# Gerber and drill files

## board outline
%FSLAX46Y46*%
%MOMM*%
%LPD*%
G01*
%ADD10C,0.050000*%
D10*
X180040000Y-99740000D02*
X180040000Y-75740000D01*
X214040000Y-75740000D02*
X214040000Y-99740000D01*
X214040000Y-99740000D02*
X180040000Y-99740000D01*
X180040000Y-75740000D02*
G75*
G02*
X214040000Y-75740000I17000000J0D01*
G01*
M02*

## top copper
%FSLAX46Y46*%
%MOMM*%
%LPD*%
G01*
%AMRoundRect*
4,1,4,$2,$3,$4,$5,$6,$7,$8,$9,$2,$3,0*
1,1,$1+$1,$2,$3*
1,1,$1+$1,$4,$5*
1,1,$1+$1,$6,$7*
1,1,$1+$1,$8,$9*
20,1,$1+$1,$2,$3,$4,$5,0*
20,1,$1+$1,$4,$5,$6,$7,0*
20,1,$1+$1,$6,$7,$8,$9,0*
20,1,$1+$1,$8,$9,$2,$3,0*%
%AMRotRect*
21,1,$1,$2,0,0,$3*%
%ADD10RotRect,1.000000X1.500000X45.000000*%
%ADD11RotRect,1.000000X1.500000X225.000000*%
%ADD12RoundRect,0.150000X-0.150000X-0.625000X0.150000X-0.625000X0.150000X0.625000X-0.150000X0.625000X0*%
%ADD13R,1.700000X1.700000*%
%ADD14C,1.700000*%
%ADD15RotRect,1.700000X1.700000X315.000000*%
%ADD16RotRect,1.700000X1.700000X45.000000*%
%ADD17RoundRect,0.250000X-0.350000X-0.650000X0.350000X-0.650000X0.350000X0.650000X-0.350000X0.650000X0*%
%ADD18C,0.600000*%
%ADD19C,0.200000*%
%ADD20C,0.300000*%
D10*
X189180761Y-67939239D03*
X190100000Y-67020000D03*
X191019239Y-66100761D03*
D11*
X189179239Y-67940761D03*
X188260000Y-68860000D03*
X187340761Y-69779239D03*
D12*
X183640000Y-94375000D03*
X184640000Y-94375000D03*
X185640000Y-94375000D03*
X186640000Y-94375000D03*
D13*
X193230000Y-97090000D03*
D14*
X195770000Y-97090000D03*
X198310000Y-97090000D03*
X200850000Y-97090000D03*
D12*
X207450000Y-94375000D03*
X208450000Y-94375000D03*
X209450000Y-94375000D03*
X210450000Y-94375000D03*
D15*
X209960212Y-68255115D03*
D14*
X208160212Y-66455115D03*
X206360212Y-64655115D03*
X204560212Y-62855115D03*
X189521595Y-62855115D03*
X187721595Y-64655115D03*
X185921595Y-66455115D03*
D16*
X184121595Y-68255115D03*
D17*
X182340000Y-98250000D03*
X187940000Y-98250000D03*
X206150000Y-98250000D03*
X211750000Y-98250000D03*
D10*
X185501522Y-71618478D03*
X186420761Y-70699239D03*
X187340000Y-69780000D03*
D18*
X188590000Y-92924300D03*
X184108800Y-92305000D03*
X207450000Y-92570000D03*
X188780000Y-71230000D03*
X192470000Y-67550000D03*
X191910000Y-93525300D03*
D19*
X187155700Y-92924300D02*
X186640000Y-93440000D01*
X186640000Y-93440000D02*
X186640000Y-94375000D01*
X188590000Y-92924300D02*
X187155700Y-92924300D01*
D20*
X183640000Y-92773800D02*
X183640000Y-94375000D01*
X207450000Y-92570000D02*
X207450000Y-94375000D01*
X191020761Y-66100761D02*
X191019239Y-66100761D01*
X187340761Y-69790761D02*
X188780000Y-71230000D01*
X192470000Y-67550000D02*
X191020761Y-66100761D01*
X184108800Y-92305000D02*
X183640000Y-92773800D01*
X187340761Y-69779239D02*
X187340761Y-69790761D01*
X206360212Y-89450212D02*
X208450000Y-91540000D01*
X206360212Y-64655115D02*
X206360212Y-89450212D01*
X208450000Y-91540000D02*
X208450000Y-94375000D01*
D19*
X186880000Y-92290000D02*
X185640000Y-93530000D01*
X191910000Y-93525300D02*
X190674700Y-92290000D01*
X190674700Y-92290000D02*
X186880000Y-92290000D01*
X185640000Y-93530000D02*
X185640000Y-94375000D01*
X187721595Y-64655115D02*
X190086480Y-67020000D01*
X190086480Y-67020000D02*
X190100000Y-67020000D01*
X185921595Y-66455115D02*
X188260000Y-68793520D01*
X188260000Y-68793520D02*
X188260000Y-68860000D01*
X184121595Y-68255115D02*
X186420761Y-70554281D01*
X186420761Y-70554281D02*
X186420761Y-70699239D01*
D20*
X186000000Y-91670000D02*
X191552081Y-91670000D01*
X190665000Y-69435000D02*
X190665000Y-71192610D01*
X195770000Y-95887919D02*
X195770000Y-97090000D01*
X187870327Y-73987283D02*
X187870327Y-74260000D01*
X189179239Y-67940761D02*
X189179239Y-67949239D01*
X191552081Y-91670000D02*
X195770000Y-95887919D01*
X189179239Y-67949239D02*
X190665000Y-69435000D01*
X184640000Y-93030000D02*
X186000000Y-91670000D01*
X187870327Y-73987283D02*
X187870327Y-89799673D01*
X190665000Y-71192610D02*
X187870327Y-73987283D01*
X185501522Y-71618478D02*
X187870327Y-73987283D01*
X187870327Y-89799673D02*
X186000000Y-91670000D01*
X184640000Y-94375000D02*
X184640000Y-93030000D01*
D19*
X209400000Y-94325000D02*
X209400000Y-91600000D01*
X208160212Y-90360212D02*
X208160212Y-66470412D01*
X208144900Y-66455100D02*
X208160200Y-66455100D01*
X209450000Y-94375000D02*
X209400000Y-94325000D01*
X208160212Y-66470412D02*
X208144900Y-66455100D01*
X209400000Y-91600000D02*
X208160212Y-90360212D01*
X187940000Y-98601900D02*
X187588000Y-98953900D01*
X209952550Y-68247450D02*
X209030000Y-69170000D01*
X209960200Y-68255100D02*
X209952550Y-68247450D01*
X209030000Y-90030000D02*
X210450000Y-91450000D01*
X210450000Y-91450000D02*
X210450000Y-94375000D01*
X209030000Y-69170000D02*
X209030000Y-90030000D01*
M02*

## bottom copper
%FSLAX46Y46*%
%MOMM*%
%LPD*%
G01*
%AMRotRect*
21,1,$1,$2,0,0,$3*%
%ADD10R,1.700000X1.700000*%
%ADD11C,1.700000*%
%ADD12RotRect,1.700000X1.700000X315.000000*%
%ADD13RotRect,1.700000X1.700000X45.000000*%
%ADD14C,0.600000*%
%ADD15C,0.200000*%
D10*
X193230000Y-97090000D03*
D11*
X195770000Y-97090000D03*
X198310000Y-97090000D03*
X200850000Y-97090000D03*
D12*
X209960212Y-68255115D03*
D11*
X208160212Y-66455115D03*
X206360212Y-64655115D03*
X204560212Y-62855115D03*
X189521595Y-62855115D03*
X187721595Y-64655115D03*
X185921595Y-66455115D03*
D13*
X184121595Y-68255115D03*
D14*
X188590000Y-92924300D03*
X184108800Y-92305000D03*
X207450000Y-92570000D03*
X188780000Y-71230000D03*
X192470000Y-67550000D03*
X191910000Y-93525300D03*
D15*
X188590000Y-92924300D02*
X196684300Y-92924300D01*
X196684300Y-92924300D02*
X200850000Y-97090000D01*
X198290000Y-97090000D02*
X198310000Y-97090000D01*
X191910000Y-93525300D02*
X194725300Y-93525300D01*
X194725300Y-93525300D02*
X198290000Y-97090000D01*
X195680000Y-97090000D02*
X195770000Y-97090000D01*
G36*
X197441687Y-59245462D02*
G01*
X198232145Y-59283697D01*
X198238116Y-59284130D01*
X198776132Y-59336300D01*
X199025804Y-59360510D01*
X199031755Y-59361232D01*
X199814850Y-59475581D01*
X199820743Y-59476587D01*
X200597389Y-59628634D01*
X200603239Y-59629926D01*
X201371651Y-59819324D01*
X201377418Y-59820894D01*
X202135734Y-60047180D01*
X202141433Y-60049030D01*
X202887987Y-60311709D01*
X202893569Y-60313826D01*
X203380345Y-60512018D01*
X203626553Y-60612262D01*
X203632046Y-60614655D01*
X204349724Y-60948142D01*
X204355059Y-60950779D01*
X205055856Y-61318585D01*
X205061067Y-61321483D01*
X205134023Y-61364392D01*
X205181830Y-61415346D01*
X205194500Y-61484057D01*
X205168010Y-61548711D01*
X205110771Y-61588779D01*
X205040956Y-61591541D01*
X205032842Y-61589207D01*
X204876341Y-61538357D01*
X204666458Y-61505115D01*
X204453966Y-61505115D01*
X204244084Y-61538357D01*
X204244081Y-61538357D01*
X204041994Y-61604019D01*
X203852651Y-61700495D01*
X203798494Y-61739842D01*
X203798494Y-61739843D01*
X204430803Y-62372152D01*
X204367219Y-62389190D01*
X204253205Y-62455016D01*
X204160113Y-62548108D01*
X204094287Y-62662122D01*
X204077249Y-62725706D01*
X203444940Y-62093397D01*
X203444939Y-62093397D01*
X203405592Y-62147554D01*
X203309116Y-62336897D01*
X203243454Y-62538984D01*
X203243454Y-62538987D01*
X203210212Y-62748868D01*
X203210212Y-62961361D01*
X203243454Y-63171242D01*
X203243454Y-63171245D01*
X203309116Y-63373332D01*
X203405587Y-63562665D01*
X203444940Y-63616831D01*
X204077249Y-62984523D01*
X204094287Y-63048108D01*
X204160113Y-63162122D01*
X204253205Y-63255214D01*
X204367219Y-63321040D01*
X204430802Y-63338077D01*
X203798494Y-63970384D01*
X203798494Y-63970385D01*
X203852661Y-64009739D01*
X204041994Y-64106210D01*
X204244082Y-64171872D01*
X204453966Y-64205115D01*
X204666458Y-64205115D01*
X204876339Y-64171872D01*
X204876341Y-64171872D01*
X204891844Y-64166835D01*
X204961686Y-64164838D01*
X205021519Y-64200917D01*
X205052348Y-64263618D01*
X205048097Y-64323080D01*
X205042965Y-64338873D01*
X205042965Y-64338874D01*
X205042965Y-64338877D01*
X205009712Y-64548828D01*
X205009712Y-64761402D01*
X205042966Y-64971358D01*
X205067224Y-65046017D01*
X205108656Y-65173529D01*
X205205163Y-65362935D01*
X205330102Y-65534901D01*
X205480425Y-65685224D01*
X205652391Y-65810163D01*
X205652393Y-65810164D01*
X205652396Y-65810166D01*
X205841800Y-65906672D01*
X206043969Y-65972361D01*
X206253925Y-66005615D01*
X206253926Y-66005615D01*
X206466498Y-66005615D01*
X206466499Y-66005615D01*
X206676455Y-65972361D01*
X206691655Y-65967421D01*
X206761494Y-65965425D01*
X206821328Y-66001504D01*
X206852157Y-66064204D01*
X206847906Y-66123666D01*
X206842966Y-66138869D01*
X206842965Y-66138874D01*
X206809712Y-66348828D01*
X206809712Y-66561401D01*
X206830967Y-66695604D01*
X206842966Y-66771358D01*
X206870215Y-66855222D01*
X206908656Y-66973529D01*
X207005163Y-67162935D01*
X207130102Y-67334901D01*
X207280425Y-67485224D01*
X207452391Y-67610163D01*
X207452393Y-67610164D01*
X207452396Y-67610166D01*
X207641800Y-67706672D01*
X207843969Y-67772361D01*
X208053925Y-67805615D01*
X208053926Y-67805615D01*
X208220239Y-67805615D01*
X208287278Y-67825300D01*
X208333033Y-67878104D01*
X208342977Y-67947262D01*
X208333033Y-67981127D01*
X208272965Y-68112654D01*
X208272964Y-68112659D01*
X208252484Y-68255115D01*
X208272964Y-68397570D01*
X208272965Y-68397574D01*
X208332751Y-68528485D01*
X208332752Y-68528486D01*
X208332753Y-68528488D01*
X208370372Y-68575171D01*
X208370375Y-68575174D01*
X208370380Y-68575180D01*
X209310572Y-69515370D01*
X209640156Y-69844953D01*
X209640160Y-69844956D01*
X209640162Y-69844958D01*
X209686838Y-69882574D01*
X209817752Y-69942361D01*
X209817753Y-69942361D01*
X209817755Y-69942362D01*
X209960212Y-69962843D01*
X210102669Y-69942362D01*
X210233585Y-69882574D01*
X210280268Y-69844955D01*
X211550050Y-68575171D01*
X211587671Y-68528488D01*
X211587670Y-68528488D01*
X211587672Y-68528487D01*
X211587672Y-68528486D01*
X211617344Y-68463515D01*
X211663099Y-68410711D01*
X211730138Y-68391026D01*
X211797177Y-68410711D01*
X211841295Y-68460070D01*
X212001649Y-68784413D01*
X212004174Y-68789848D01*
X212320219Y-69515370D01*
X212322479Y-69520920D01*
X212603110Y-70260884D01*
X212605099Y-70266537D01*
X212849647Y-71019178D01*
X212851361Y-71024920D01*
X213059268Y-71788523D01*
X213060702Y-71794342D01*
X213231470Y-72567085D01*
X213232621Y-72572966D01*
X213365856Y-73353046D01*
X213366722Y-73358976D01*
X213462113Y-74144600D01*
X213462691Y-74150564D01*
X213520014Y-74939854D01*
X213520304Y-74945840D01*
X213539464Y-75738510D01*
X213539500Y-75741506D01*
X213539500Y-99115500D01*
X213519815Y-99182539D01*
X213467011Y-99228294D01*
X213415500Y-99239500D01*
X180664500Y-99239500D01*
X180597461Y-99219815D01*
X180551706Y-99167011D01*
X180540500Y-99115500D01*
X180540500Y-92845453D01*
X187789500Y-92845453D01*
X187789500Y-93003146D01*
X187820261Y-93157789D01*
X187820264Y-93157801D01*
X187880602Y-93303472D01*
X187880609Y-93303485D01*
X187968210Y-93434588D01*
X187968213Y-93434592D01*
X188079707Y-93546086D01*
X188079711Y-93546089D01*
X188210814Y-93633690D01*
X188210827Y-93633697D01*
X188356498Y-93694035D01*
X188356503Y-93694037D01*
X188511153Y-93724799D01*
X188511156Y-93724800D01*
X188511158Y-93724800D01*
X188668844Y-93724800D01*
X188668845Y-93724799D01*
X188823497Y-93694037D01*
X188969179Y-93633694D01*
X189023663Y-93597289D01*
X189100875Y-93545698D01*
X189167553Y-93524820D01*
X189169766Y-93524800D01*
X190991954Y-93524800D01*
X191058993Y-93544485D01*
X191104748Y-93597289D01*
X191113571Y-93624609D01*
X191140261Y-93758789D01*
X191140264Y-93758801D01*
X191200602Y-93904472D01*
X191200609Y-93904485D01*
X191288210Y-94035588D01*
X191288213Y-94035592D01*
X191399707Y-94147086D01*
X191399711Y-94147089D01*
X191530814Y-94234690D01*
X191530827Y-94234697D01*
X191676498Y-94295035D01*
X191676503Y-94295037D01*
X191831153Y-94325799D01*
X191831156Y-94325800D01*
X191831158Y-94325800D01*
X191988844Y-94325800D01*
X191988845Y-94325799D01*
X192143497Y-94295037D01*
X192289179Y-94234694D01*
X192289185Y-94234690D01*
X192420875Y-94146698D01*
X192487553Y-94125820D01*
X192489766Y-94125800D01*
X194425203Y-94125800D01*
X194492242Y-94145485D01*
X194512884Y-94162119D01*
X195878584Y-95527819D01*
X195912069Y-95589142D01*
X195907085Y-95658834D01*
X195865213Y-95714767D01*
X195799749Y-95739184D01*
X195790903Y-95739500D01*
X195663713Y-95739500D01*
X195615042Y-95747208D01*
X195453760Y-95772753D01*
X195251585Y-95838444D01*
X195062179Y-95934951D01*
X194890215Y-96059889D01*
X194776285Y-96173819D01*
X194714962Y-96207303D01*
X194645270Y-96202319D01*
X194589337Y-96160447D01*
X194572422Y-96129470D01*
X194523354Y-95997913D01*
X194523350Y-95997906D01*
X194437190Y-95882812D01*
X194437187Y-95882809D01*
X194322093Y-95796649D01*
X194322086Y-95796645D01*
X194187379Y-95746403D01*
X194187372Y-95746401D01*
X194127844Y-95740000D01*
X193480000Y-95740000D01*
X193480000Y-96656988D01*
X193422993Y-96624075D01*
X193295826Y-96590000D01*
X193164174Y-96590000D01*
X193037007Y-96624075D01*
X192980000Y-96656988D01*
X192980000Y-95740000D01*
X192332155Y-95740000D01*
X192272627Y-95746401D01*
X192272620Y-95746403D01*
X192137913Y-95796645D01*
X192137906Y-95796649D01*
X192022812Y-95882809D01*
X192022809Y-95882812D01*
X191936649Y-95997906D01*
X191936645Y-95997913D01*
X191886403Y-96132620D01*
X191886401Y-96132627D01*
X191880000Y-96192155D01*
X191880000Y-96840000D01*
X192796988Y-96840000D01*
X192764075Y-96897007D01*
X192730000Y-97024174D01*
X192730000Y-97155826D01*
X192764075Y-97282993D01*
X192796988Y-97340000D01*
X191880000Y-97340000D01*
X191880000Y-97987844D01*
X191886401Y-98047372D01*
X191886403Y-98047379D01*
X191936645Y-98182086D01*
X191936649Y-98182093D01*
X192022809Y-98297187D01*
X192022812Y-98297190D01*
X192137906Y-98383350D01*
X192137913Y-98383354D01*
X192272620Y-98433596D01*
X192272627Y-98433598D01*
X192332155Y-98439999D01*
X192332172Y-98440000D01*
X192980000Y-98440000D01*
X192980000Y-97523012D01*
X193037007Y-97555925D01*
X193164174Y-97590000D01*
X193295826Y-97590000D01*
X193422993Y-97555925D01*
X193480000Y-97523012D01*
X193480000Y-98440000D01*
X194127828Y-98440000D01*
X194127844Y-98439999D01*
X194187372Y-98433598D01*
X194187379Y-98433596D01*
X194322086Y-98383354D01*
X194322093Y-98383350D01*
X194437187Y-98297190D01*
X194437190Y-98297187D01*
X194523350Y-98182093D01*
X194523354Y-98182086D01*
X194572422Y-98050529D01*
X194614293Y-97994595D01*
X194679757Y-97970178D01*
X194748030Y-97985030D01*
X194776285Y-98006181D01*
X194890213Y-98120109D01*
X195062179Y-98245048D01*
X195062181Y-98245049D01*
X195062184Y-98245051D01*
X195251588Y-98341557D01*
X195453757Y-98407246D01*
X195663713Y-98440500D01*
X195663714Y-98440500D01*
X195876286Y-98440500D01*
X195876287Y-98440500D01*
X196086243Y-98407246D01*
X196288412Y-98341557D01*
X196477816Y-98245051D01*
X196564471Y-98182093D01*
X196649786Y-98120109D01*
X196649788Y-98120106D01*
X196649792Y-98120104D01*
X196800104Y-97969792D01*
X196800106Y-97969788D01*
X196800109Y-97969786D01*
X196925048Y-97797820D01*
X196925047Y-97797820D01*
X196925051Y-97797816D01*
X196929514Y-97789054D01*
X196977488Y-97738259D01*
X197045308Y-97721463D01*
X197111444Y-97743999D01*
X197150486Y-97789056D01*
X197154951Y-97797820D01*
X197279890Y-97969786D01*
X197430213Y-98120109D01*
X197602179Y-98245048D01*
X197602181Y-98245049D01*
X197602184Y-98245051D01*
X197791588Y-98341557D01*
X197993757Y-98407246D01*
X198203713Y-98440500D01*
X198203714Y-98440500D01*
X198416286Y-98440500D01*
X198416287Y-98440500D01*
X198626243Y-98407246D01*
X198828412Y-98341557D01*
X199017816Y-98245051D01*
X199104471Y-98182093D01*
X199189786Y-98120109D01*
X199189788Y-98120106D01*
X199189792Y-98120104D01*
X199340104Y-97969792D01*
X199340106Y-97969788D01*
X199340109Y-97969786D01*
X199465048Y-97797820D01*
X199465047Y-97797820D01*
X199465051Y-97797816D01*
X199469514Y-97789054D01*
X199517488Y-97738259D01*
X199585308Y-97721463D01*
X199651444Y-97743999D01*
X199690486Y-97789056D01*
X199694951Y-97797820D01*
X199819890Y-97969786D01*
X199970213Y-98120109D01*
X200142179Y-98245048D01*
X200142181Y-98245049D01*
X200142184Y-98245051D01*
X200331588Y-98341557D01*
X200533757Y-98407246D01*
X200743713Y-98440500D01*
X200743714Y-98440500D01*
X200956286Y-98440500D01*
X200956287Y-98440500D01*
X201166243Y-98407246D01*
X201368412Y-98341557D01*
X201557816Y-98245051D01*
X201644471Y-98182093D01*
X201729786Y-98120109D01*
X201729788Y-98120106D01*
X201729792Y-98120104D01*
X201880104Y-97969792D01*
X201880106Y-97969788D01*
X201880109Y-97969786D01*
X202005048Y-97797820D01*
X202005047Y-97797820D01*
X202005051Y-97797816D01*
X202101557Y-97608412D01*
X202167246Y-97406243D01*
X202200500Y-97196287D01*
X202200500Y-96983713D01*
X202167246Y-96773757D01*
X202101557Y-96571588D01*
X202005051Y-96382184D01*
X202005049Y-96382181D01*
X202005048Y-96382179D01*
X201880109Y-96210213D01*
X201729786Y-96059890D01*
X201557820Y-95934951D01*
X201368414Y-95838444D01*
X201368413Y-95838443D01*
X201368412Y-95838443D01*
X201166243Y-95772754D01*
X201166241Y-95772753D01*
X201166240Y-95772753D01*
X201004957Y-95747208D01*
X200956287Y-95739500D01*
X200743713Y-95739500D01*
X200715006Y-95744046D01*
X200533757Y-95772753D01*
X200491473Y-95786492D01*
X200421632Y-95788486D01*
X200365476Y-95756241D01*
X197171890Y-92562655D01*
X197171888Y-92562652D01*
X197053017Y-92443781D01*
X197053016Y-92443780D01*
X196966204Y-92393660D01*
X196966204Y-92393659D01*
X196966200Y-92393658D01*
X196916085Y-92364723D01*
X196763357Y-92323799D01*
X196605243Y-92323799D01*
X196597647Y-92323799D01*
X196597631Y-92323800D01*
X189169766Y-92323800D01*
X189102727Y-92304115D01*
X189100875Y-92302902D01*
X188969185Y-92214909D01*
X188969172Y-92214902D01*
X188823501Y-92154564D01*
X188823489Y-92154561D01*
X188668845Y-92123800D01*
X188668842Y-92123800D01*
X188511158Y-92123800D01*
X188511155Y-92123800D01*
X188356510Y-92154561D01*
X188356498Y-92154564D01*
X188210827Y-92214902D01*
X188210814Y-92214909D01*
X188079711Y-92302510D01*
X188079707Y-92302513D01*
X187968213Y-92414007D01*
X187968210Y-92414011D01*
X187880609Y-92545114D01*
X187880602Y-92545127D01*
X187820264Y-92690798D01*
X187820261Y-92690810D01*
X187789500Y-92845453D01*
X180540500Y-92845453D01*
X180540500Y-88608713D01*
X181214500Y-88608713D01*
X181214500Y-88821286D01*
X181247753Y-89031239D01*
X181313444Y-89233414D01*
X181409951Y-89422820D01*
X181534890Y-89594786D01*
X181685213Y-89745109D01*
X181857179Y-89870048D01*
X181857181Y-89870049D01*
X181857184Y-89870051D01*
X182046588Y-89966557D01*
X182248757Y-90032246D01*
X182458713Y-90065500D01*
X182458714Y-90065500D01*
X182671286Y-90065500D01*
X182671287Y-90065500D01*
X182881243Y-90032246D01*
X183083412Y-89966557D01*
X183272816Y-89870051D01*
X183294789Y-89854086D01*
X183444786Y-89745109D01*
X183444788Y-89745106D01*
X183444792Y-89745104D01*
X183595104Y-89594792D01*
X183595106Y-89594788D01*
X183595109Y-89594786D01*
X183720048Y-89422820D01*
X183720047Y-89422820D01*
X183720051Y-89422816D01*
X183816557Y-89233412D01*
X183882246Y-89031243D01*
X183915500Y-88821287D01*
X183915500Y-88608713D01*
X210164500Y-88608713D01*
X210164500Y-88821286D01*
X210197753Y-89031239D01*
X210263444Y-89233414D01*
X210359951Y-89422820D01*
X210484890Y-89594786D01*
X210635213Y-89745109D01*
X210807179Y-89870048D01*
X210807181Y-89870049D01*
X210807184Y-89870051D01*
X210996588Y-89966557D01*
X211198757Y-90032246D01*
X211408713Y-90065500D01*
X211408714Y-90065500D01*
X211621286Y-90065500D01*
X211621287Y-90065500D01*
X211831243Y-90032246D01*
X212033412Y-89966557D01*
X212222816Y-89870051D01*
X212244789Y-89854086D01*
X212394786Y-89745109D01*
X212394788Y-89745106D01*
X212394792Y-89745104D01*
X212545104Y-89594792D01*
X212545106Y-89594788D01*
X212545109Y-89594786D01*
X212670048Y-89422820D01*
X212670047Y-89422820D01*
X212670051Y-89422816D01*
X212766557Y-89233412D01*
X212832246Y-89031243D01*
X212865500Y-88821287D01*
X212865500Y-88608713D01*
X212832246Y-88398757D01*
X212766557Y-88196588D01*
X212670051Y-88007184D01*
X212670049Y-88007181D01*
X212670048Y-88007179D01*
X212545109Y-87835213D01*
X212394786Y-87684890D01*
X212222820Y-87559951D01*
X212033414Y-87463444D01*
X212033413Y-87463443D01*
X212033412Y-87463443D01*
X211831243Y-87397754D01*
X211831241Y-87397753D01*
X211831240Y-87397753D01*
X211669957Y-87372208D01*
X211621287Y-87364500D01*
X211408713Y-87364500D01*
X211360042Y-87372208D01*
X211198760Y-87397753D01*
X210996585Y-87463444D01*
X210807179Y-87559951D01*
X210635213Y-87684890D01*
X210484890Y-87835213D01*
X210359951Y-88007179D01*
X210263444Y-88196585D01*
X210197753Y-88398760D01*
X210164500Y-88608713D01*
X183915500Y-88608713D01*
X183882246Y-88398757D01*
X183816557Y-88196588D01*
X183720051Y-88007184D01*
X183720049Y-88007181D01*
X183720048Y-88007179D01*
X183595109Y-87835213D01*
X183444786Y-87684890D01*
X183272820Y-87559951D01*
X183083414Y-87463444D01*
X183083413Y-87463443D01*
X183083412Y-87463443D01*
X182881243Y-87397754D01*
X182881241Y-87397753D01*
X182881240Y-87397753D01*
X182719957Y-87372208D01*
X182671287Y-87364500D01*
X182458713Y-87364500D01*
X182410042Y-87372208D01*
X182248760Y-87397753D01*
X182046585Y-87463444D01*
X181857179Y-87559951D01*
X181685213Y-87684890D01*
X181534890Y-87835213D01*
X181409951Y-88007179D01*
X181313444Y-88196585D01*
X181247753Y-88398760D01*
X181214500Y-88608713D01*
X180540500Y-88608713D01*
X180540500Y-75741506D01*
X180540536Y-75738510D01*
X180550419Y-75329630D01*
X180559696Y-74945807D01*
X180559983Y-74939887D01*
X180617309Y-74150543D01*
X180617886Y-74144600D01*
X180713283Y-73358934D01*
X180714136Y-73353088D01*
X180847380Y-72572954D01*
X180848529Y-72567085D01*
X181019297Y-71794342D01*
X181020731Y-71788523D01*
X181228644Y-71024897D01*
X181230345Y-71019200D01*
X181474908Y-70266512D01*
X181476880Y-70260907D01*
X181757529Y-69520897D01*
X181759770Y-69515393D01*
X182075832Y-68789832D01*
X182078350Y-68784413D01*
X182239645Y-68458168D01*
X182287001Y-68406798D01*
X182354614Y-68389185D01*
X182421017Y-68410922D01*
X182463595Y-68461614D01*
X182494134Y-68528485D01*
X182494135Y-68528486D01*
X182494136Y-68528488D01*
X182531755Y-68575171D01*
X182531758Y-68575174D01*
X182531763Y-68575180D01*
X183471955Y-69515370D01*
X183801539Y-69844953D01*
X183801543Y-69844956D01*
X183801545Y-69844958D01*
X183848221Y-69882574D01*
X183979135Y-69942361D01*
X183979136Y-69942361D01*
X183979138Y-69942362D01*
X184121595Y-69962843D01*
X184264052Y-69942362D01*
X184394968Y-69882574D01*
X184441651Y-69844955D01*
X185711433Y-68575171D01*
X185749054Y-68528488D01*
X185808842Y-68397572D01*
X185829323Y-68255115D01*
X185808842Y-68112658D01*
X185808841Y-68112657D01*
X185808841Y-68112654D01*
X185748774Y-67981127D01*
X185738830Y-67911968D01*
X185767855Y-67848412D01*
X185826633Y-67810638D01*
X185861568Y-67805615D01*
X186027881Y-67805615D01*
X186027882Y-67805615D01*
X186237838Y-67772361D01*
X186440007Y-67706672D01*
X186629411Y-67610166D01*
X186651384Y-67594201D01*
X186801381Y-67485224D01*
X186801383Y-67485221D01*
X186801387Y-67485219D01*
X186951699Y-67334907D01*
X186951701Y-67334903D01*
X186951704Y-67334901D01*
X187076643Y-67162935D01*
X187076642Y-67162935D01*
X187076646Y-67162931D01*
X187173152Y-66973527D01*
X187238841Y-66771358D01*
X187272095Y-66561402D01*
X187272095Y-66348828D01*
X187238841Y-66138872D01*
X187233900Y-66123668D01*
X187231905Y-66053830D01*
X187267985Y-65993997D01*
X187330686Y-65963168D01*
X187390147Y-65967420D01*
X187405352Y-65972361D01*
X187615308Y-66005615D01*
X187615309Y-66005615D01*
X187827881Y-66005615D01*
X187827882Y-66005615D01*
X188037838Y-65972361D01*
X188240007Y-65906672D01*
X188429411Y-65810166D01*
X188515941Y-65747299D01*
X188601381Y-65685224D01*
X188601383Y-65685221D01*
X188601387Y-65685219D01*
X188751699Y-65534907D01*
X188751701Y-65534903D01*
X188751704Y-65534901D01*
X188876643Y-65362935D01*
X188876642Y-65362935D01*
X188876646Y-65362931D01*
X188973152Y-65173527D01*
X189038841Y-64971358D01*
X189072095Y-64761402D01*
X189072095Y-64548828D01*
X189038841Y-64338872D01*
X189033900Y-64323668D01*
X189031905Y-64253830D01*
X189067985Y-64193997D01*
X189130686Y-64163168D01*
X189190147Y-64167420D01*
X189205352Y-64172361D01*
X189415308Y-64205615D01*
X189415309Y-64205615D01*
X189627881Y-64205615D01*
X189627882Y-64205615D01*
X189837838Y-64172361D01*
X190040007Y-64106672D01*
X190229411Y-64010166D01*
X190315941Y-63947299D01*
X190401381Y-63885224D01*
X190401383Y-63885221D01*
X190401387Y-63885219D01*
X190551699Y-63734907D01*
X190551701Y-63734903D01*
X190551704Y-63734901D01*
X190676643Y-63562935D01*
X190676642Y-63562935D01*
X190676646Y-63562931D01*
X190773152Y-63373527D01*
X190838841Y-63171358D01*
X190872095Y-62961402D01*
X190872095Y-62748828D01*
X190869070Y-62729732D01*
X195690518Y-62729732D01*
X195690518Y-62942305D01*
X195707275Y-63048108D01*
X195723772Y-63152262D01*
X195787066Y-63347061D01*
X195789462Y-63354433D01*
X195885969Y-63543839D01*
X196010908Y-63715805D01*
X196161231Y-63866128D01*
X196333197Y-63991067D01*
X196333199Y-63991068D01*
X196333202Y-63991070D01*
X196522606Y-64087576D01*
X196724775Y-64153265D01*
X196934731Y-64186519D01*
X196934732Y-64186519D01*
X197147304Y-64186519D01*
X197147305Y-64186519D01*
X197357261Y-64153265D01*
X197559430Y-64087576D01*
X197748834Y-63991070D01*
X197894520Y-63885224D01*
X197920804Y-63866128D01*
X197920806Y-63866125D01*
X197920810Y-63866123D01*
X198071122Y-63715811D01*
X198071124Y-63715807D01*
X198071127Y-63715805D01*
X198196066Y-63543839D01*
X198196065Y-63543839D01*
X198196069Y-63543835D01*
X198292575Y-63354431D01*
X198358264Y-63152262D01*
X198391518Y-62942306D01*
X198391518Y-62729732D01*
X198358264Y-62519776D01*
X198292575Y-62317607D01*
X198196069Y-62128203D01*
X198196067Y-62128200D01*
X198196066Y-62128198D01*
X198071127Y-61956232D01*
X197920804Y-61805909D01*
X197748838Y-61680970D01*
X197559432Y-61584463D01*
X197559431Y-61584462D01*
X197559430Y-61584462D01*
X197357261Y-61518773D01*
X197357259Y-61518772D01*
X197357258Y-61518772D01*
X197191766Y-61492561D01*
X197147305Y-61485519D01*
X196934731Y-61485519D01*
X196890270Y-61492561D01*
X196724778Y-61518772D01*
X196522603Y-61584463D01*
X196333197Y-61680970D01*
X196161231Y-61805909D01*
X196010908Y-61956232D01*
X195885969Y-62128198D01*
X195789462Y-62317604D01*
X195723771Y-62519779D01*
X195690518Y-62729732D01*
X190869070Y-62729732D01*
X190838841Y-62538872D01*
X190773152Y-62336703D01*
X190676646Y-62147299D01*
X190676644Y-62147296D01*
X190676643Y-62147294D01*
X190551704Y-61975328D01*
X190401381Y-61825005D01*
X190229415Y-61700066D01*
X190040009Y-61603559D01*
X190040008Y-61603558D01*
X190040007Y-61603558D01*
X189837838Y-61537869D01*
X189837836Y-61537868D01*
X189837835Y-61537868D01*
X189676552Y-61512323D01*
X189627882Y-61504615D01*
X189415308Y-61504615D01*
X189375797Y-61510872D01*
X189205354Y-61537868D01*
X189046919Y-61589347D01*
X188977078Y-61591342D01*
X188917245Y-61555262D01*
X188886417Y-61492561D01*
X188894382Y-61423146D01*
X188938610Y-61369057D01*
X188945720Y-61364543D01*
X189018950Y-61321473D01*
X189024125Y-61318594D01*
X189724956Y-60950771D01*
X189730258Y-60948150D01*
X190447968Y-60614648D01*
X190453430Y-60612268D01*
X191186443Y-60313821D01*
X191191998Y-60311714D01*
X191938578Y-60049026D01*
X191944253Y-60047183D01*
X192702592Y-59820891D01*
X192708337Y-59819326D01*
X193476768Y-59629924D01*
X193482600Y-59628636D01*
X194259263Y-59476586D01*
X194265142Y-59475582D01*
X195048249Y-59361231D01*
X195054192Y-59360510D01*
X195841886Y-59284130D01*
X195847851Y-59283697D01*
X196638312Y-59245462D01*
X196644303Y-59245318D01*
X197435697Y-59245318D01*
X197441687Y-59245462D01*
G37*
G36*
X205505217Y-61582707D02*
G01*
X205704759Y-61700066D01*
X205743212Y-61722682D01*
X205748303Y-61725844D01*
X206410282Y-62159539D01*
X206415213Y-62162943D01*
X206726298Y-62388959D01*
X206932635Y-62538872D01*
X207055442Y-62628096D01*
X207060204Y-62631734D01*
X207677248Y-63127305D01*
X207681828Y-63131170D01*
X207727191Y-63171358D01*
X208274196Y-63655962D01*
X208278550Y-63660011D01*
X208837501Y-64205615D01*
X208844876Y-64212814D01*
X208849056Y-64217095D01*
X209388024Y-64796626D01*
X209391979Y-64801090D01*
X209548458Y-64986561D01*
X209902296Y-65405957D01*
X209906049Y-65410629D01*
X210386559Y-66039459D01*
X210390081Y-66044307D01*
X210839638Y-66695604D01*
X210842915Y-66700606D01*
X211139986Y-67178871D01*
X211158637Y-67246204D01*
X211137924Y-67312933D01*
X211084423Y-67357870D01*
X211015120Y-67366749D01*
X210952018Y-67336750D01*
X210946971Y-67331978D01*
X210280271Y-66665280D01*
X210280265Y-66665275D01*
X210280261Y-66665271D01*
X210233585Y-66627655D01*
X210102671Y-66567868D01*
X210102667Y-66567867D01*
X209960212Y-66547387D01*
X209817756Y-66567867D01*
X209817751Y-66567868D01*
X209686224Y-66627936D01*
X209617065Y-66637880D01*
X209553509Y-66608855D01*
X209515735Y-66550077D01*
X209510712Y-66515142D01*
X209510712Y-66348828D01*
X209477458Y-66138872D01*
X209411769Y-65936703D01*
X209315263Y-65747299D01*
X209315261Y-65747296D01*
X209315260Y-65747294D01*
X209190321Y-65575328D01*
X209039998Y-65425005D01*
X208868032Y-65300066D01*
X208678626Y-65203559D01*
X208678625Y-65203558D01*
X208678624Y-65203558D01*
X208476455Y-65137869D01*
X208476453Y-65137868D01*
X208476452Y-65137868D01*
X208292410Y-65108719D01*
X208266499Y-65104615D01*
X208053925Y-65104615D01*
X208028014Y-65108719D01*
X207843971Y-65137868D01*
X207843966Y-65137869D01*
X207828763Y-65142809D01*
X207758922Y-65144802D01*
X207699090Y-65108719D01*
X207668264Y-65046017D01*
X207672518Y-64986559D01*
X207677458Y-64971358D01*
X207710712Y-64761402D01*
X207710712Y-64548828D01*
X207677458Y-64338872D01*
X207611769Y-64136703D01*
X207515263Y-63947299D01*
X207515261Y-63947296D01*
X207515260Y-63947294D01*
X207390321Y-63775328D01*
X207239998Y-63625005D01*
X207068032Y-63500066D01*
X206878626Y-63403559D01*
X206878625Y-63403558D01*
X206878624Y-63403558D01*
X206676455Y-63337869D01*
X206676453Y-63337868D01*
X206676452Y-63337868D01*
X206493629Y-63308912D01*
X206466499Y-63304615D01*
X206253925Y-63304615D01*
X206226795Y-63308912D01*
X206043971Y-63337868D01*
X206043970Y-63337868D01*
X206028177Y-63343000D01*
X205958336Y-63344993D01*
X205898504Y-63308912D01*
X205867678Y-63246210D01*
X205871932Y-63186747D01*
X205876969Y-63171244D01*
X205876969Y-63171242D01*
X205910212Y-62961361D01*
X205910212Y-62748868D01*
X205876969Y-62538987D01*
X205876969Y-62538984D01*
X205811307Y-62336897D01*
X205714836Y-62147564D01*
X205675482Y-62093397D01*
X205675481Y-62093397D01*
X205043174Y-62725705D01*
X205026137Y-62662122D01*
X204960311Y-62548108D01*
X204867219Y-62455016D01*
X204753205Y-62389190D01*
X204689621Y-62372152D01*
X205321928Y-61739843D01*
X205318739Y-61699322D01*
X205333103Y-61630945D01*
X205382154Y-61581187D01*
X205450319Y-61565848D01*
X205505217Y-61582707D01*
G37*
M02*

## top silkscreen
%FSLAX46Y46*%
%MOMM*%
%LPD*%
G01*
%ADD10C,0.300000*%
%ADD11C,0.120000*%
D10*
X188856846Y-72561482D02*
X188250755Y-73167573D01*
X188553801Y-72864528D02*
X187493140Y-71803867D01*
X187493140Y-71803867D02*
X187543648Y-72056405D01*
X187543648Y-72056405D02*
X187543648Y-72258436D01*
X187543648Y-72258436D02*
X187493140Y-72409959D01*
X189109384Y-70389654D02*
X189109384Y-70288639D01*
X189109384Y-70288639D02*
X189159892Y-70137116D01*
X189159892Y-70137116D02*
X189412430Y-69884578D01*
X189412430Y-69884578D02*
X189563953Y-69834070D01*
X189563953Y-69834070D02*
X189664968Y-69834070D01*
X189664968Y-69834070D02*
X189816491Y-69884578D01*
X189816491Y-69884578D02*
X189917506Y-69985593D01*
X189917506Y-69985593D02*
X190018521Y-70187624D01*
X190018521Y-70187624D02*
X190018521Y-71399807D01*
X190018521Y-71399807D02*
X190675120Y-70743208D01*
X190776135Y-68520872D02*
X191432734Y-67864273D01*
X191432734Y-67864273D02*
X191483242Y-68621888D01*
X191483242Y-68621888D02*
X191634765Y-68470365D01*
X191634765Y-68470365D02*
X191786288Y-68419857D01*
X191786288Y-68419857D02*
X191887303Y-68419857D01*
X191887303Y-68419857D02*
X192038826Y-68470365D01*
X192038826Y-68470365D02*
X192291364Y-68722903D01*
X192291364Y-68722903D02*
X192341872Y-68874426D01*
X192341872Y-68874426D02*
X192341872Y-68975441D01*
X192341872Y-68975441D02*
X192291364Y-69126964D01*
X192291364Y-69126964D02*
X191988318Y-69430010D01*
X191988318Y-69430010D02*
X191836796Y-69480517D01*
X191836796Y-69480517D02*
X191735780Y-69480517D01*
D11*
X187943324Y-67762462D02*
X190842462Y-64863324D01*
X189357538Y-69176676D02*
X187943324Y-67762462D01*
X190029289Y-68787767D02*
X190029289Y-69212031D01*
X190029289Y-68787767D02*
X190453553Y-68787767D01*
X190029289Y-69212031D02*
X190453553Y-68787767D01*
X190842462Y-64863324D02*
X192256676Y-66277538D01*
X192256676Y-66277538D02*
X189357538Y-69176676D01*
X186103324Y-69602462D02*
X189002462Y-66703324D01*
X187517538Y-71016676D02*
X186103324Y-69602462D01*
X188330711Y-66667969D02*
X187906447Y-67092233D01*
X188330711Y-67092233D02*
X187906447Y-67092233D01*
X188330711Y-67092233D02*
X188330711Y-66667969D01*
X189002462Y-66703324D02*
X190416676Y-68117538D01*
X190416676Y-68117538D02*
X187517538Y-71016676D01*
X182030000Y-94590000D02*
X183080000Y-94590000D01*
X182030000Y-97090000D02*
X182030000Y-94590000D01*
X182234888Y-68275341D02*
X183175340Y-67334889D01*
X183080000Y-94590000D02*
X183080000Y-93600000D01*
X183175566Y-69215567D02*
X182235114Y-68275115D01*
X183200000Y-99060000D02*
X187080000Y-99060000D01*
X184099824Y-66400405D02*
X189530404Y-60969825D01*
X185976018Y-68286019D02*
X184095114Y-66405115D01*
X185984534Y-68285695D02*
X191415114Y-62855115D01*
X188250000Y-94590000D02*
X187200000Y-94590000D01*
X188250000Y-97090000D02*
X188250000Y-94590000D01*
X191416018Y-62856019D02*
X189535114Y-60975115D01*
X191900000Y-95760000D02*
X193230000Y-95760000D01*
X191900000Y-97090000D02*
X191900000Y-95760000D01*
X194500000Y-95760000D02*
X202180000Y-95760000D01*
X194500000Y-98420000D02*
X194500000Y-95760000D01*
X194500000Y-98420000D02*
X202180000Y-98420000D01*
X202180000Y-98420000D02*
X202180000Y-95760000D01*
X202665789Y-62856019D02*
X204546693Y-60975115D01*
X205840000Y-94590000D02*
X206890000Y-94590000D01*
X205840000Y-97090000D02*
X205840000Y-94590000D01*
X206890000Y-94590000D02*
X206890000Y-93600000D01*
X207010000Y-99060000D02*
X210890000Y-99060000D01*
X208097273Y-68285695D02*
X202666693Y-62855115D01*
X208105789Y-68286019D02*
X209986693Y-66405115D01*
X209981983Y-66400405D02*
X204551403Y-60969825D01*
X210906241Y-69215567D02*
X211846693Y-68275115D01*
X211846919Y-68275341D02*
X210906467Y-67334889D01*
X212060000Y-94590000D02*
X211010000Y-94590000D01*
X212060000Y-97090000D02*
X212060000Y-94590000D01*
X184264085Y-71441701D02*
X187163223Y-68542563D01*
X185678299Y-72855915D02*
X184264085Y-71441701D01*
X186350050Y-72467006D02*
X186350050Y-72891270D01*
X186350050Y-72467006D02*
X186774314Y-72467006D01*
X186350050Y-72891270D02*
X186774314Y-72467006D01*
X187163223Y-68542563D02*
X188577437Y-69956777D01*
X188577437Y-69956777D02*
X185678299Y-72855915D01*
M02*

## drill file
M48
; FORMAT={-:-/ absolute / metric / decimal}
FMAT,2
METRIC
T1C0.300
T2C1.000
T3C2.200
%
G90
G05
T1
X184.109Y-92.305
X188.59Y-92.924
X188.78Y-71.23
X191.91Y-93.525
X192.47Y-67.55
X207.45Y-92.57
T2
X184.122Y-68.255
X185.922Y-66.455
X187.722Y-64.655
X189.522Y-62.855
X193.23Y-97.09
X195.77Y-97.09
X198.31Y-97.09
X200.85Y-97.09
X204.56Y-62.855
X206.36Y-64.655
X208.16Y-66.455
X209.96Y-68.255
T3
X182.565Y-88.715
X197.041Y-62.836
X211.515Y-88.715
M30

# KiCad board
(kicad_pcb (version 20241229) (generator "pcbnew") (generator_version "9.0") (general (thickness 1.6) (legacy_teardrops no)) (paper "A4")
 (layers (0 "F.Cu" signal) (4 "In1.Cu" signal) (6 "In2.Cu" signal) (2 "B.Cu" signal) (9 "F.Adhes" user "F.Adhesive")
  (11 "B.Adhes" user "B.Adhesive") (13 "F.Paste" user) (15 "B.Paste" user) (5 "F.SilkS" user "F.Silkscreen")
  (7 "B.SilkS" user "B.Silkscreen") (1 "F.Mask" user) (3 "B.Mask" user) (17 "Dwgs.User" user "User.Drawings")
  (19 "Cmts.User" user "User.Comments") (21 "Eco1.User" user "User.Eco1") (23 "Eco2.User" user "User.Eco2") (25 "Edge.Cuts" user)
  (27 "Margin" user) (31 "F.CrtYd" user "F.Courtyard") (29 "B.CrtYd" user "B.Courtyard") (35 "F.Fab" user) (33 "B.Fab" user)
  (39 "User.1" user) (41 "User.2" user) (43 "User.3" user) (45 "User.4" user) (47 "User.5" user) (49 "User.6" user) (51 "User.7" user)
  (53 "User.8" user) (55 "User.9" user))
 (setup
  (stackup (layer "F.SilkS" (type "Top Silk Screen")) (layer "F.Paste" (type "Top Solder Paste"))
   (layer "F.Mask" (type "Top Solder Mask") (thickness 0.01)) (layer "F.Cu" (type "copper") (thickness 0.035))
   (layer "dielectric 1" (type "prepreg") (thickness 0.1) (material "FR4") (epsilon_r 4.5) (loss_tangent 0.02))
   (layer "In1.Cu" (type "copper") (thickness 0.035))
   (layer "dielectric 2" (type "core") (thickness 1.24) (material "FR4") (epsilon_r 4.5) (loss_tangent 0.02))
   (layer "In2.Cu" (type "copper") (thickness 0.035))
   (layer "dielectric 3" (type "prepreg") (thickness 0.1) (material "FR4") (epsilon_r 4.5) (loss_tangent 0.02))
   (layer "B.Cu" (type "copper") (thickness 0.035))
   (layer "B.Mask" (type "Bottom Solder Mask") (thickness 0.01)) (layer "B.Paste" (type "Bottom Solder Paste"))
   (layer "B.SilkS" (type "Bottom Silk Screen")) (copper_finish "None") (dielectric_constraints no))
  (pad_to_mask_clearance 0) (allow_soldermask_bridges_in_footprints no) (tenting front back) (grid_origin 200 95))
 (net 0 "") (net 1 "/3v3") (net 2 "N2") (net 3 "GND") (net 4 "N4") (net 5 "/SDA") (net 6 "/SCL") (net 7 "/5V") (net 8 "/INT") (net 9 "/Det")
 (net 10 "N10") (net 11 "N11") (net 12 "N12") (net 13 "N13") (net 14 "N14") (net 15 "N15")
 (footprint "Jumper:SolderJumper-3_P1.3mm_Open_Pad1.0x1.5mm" (layer "F.Cu") (at 190.1 67.02 45)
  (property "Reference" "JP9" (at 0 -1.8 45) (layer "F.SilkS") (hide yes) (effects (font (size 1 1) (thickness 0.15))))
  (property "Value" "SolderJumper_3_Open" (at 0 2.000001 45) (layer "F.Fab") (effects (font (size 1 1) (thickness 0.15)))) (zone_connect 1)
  (fp_line (start -2.05 -1) (end 2.05 -1) (stroke (width 0.12) (type solid)) (layer "F.SilkS"))
  (fp_line (start -2.05 1) (end -2.05 -1) (stroke (width 0.12) (type solid)) (layer "F.SilkS"))
  (fp_line (start -1.3 1.2) (end -1.6 1.5) (stroke (width 0.12) (type solid)) (layer "F.SilkS"))
  (fp_line (start -1.3 1.2) (end -1 1.5) (stroke (width 0.12) (type solid)) (layer "F.SilkS"))
  (fp_line (start -1.6 1.5) (end -1 1.5) (stroke (width 0.12) (type solid)) (layer "F.SilkS"))
  (fp_line (start 2.05 -1) (end 2.05 1) (stroke (width 0.12) (type solid)) (layer "F.SilkS"))
  (fp_line (start 2.05 1) (end -2.05 1) (stroke (width 0.12) (type solid)) (layer "F.SilkS"))
  (pad "1" smd rect (at -1.3 0 45) (size 1 1.5) (layers "F.Cu" "F.Mask") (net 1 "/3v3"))
  (pad "2" smd rect (at 0 0 45) (size 1 1.5) (layers "F.Cu" "F.Mask") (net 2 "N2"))
  (pad "3" smd rect (at 1.3 0 45) (size 1 1.5) (layers "F.Cu" "F.Mask") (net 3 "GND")))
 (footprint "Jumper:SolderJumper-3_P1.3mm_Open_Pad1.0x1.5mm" (layer "F.Cu") (at 188.26 68.86 -135)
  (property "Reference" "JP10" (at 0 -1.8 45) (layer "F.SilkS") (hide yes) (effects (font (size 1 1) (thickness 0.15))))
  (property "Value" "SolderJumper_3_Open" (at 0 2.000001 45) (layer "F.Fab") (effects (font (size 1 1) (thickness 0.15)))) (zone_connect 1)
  (fp_line (start 2.05 1) (end -2.05 1) (stroke (width 0.12) (type solid)) (layer "F.SilkS"))
  (fp_line (start 2.05 -1) (end 2.05 1) (stroke (width 0.12) (type solid)) (layer "F.SilkS"))
  (fp_line (start -1.6 1.5) (end -1 1.5) (stroke (width 0.12) (type solid)) (layer "F.SilkS"))
  (fp_line (start -1.3 1.2) (end -1 1.5) (stroke (width 0.12) (type solid)) (layer "F.SilkS"))
  (fp_line (start -1.3 1.2) (end -1.6 1.5) (stroke (width 0.12) (type solid)) (layer "F.SilkS"))
  (fp_line (start -2.05 1) (end -2.05 -1) (stroke (width 0.12) (type solid)) (layer "F.SilkS"))
  (fp_line (start -2.05 -1) (end 2.05 -1) (stroke (width 0.12) (type solid)) (layer "F.SilkS"))
  (pad "1" smd rect (at -1.3 0 225) (size 1 1.5) (layers "F.Cu" "F.Mask") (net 1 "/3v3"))
  (pad "2" smd rect (at 0 0 225) (size 1 1.5) (layers "F.Cu" "F.Mask") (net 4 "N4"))
  (pad "3" smd rect (at 1.3 0 225) (size 1 1.5) (layers "F.Cu" "F.Mask") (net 3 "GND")))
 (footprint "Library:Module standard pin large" (layer "F.Cu") (at 197.04 75.74)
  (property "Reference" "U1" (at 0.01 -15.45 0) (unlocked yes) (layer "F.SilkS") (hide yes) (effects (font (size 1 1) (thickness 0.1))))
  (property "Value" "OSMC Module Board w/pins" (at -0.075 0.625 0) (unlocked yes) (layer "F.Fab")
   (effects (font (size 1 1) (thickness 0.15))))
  (fp_line (start -15.01 18.85) (end -13.96 18.85) (stroke (width 0.12) (type solid)) (layer "F.SilkS"))
  (fp_line (start -15.01 21.35) (end -15.01 18.85) (stroke (width 0.12) (type solid)) (layer "F.SilkS"))
  (fp_line (start -14.805112 -7.464659) (end -13.86466 -8.405111) (stroke (width 0.12) (type solid)) (layer "F.SilkS"))
  (fp_line (start -13.96 18.85) (end -13.96 17.86) (stroke (width 0.12) (type solid)) (layer "F.SilkS"))
  (fp_line (start -13.864434 -6.524433) (end -14.804886 -7.464885) (stroke (width 0.12) (type solid)) (layer "F.SilkS"))
  (fp_line (start -13.84 23.32) (end -9.96 23.32) (stroke (width 0.12) (type solid)) (layer "F.SilkS"))
  (fp_line (start -12.940176 -9.339595) (end -7.509596 -14.770175) (stroke (width 0.12) (type solid)) (layer "F.SilkS"))
  (fp_line (start -11.063982 -7.453981) (end -12.944886 -9.334885) (stroke (width 0.12) (type solid)) (layer "F.SilkS"))
  (fp_line (start -11.055466 -7.454305) (end -5.624886 -12.884885) (stroke (width 0.12) (type solid)) (layer "F.SilkS"))
  (fp_line (start -8.79 18.85) (end -9.84 18.85) (stroke (width 0.12) (type solid)) (layer "F.SilkS"))
  (fp_line (start -8.79 21.35) (end -8.79 18.85) (stroke (width 0.12) (type solid)) (layer "F.SilkS"))
  (fp_line (start -5.623982 -12.883981) (end -7.504886 -14.764885) (stroke (width 0.12) (type solid)) (layer "F.SilkS"))
  (fp_line (start -5.14 20.02) (end -3.81 20.02) (stroke (width 0.12) (type solid)) (layer "F.SilkS"))
  (fp_line (start -5.14 21.35) (end -5.14 20.02) (stroke (width 0.12) (type solid)) (layer "F.SilkS"))
  (fp_line (start -2.54 20.02) (end 5.14 20.02) (stroke (width 0.12) (type solid)) (layer "F.SilkS"))
  (fp_line (start -2.54 22.68) (end -2.54 20.02) (stroke (width 0.12) (type solid)) (layer "F.SilkS"))
  (fp_line (start -2.54 22.68) (end 5.14 22.68) (stroke (width 0.12) (type solid)) (layer "F.SilkS"))
  (fp_line (start 5.14 22.68) (end 5.14 20.02) (stroke (width 0.12) (type solid)) (layer "F.SilkS"))
  (fp_line (start 5.625789 -12.883981) (end 7.506693 -14.764885) (stroke (width 0.12) (type solid)) (layer "F.SilkS"))
  (fp_line (start 8.8 18.85) (end 9.85 18.85) (stroke (width 0.12) (type solid)) (layer "F.SilkS"))
  (fp_line (start 8.8 21.35) (end 8.8 18.85) (stroke (width 0.12) (type solid)) (layer "F.SilkS"))
  (fp_line (start 9.85 18.85) (end 9.85 17.86) (stroke (width 0.12) (type solid)) (layer "F.SilkS"))
  (fp_line (start 9.97 23.32) (end 13.85 23.32) (stroke (width 0.12) (type solid)) (layer "F.SilkS"))
  (fp_line (start 11.057273 -7.454305) (end 5.626693 -12.884885) (stroke (width 0.12) (type solid)) (layer "F.SilkS"))
  (fp_line (start 11.065789 -7.453981) (end 12.946693 -9.334885) (stroke (width 0.12) (type solid)) (layer "F.SilkS"))
  (fp_line (start 12.941983 -9.339595) (end 7.511403 -14.770175) (stroke (width 0.12) (type solid)) (layer "F.SilkS"))
  (fp_line (start 13.866241 -6.524433) (end 14.806693 -7.464885) (stroke (width 0.12) (type solid)) (layer "F.SilkS"))
  (fp_line (start 14.806919 -7.464659) (end 13.866467 -8.405111) (stroke (width 0.12) (type solid)) (layer "F.SilkS"))
  (fp_line (start 15.02 18.85) (end 13.97 18.85) (stroke (width 0.12) (type solid)) (layer "F.SilkS"))
  (fp_line (start 15.02 21.35) (end 15.02 18.85) (stroke (width 0.12) (type solid)) (layer "F.SilkS"))
  (fp_line (start -17 24) (end -17 0) (stroke (width 0.05) (type solid)) (layer "Edge.Cuts"))
  (fp_line (start 17 0) (end 17 24) (stroke (width 0.05) (type solid)) (layer "Edge.Cuts"))
  (fp_line (start 17 24) (end -17 24) (stroke (width 0.05) (type solid)) (layer "Edge.Cuts"))
  (fp_arc (start -17 0) (mid 0 -17) (end 17 0) (stroke (width 0.05) (type solid)) (layer "Edge.Cuts"))
  (pad "" np_thru_hole circle (at -14.475 12.975) (size 2.2 2.2) (drill 2.2) (layers "*.Cu" "*.Mask"))
  (pad "" np_thru_hole circle (at 14.475 12.975) (size 2.2 2.2) (drill 2.2) (layers "*.Cu" "*.Mask"))
  (pad "1" smd roundrect (at -13.4 18.635) (size 0.6 1.55) (layers "F.Cu" "F.Mask" "F.Paste") (roundrect_rratio 0.25) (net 3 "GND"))
  (pad "2" smd roundrect (at -12.4 18.635) (size 0.6 1.55) (layers "F.Cu" "F.Mask" "F.Paste") (roundrect_rratio 0.25) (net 1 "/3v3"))
  (pad "3" smd roundrect (at -11.4 18.635) (size 0.6 1.55) (layers "F.Cu" "F.Mask" "F.Paste") (roundrect_rratio 0.25) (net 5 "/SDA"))
  (pad "4" smd roundrect (at -10.4 18.635) (size 0.6 1.55) (layers "F.Cu" "F.Mask" "F.Paste") (roundrect_rratio 0.25) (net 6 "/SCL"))
  (pad "5" thru_hole rect (at -3.81 21.35 90) (size 1.7 1.7) (drill 1) (layers "*.Cu" "*.Mask") (remove_unused_layers no) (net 3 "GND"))
  (pad "6" thru_hole circle (at -1.27 21.35 90) (size 1.7 1.7) (drill 1) (layers "*.Cu" "*.Mask") (remove_unused_layers no) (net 1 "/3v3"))
  (pad "7" thru_hole circle (at 1.27 21.35 90) (size 1.7 1.7) (drill 1) (layers "*.Cu" "*.Mask") (remove_unused_layers no) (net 5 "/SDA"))
  (pad "8" thru_hole circle (at 3.81 21.35 90) (size 1.7 1.7) (drill 1) (layers "*.Cu" "*.Mask") (remove_unused_layers no) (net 6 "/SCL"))
  (pad "9" smd roundrect (at 10.41 18.635) (size 0.6 1.55) (layers "F.Cu" "F.Mask" "F.Paste") (roundrect_rratio 0.25) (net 3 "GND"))
  (pad "10" smd roundrect (at 11.41 18.635) (size 0.6 1.55) (layers "F.Cu" "F.Mask" "F.Paste") (roundrect_rratio 0.25) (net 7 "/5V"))
  (pad "11" smd roundrect (at 12.41 18.635) (size 0.6 1.55) (layers "F.Cu" "F.Mask" "F.Paste") (roundrect_rratio 0.25) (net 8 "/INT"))
  (pad "12" smd roundrect (at 13.41 18.635) (size 0.6 1.55) (layers "F.Cu" "F.Mask" "F.Paste") (roundrect_rratio 0.25) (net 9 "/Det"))
  (pad "13" thru_hole rect (at 12.920212 -7.484885 315) (size 1.7 1.7) (drill 1) (layers "*.Cu" "*.Mask") (remove_unused_layers no)
   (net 9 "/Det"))
  (pad "14" thru_hole circle (at 11.120212 -9.284885 270) (size 1.7 1.7) (drill 1) (layers "*.Cu" "*.Mask") (remove_unused_layers no)
   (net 8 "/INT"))
  (pad "15" thru_hole circle (at 9.320212 -11.084885 270) (size 1.7 1.7) (drill 1) (layers "*.Cu" "*.Mask") (remove_unused_layers no)
   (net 7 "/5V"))
  (pad "16" thru_hole circle (at 7.520212 -12.884885 270) (size 1.7 1.7) (drill 1) (layers "*.Cu" "*.Mask") (remove_unused_layers no)
   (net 3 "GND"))
  (pad "17" thru_hole circle (at -7.518405 -12.884885 90) (size 1.7 1.7) (drill 1) (layers "*.Cu" "*.Mask") (remove_unused_layers no)
   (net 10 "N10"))
  (pad "18" thru_hole circle (at -9.318405 -11.084885 90) (size 1.7 1.7) (drill 1) (layers "*.Cu" "*.Mask") (remove_unused_layers no)
   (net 2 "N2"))
  (pad "19" thru_hole circle (at -11.118405 -9.284885 90) (size 1.7 1.7) (drill 1) (layers "*.Cu" "*.Mask") (remove_unused_layers no)
   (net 4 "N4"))
  (pad "20" thru_hole rect (at -12.918405 -7.484885 45) (size 1.7 1.7) (drill 1) (layers "*.Cu" "*.Mask") (remove_unused_layers no)
   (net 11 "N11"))
  (pad "MP" smd roundrect (at -14.7 22.51) (size 1.2 1.8) (layers "F.Cu" "F.Mask" "F.Paste") (roundrect_rratio 0.208333) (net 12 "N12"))
  (pad "MP" smd roundrect (at -9.1 22.51) (size 1.2 1.8) (layers "F.Cu" "F.Mask" "F.Paste") (roundrect_rratio 0.208333) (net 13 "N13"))
  (pad "MP" smd roundrect (at 9.11 22.51) (size 1.2 1.8) (layers "F.Cu" "F.Mask" "F.Paste") (roundrect_rratio 0.208333) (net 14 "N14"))
  (pad "MP" smd roundrect (at 14.71 22.51) (size 1.2 1.8) (layers "F.Cu" "F.Mask" "F.Paste") (roundrect_rratio 0.208333) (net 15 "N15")))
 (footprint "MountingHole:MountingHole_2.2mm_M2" (layer "F.Cu") (at 197.041018 62.836019)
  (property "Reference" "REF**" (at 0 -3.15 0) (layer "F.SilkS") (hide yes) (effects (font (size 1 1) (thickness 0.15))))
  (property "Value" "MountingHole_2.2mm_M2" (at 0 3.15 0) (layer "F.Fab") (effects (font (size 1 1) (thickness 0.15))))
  (pad "" np_thru_hole circle (at 0 0) (size 2.2 2.2) (drill 2.2) (layers "*.Cu" "*.Mask")))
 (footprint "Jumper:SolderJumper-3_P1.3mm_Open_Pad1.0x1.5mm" (layer "F.Cu") (at 186.420761 70.699239 45)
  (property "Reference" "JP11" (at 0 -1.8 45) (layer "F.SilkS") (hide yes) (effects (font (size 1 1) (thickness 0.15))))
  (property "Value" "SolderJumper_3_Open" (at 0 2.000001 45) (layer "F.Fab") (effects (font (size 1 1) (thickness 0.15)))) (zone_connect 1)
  (fp_line (start -2.05 -1) (end 2.05 -1) (stroke (width 0.12) (type solid)) (layer "F.SilkS"))
  (fp_line (start -2.05 1) (end -2.05 -1) (stroke (width 0.12) (type solid)) (layer "F.SilkS"))
  (fp_line (start -1.3 1.2) (end -1.6 1.5) (stroke (width 0.12) (type solid)) (layer "F.SilkS"))
  (fp_line (start -1.3 1.2) (end -1 1.5) (stroke (width 0.12) (type solid)) (layer "F.SilkS"))
  (fp_line (start -1.6 1.5) (end -1 1.5) (stroke (width 0.12) (type solid)) (layer "F.SilkS"))
  (fp_line (start 2.05 -1) (end 2.05 1) (stroke (width 0.12) (type solid)) (layer "F.SilkS"))
  (fp_line (start 2.05 1) (end -2.05 1) (stroke (width 0.12) (type solid)) (layer "F.SilkS"))
  (pad "1" smd rect (at -1.3 0 45) (size 1 1.5) (layers "F.Cu" "F.Mask") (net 1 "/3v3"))
  (pad "2" smd rect (at 0 0 45) (size 1 1.5) (layers "F.Cu" "F.Mask") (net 11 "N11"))
  (pad "3" smd rect (at 1.3 0 45) (size 1 1.5) (layers "F.Cu" "F.Mask") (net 3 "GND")))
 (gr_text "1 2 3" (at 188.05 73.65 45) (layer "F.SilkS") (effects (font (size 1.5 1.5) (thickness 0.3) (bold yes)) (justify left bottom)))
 (segment (start 187.1557 92.9243) (end 186.64 93.44) (width 0.2) (layer "F.Cu") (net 6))
 (segment (start 186.64 93.44) (end 186.64 94.375) (width 0.2) (layer "F.Cu") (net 6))
 (segment (start 188.59 92.9243) (end 187.1557 92.9243) (width 0.2) (layer "F.Cu") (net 6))
 (via (at 188.59 92.9243) (size 0.6) (drill 0.3) (layers "F.Cu" "B.Cu") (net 6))
 (segment (start 188.59 92.9243) (end 196.6843 92.9243) (width 0.2) (layer "B.Cu") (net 6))
 (segment (start 196.6843 92.9243) (end 200.85 97.09) (width 0.2) (layer "B.Cu") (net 6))
 (segment (start 183.64 92.7738) (end 183.64 94.375) (width 0.3) (layer "F.Cu") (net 3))
 (segment (start 207.45 92.57) (end 207.45 94.375) (width 0.3) (layer "F.Cu") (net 3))
 (segment (start 191.020761 66.100761) (end 191.019239 66.100761) (width 0.3) (layer "F.Cu") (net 3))
 (segment (start 187.340761 69.790761) (end 188.78 71.23) (width 0.3) (layer "F.Cu") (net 3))
 (segment (start 192.47 67.55) (end 191.020761 66.100761) (width 0.3) (layer "F.Cu") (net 3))
 (segment (start 184.1088 92.305) (end 183.64 92.7738) (width 0.3) (layer "F.Cu") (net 3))
 (segment (start 187.340761 69.779239) (end 187.340761 69.790761) (width 0.3) (layer "F.Cu") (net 3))
 (via (at 184.1088 92.305) (size 0.6) (drill 0.3) (layers "F.Cu" "B.Cu") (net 3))
 (via (at 207.45 92.57) (size 0.6) (drill 0.3) (layers "F.Cu" "B.Cu") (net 3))
 (via (at 188.78 71.23) (size 0.6) (drill 0.3) (layers "F.Cu" "B.Cu") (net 3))
 (via (at 192.47 67.55) (size 0.6) (drill 0.3) (layers "F.Cu" "B.Cu") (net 3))
 (segment (start 206.360212 89.450212) (end 208.45 91.54) (width 0.3) (layer "F.Cu") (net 7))
 (segment (start 206.360212 64.655115) (end 206.360212 89.450212) (width 0.3) (layer "F.Cu") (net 7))
 (segment (start 208.45 91.54) (end 208.45 94.375) (width 0.3) (layer "F.Cu") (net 7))
 (segment (start 186.88 92.29) (end 185.64 93.53) (width 0.2) (layer "F.Cu") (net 5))
 (segment (start 191.91 93.5253) (end 190.6747 92.29) (width 0.2) (layer "F.Cu") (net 5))
 (segment (start 190.6747 92.29) (end 186.88 92.29) (width 0.2) (layer "F.Cu") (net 5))
 (segment (start 185.64 93.53) (end 185.64 94.375) (width 0.2) (layer "F.Cu") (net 5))
 (via (at 191.91 93.5253) (size 0.6) (drill 0.3) (layers "F.Cu" "B.Cu") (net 5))
 (segment (start 198.29 97.09) (end 198.31 97.09) (width 0.2) (layer "B.Cu") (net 5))
 (segment (start 191.91 93.5253) (end 194.7253 93.5253) (width 0.2) (layer "B.Cu") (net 5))
 (segment (start 194.7253 93.5253) (end 198.29 97.09) (width 0.2) (layer "B.Cu") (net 5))
 (segment (start 187.721595 64.655115) (end 190.08648 67.02) (width 0.2) (layer "F.Cu") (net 2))
 (segment (start 190.08648 67.02) (end 190.1 67.02) (width 0.2) (layer "F.Cu") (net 2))
 (segment (start 185.921595 66.455115) (end 188.26 68.79352) (width 0.2) (layer "F.Cu") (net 4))
 (segment (start 188.26 68.79352) (end 188.26 68.86) (width 0.2) (layer "F.Cu") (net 4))
 (segment (start 184.121595 68.255115) (end 186.420761 70.554281) (width 0.2) (layer "F.Cu") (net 11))
 (segment (start 186.420761 70.554281) (end 186.420761 70.699239) (width 0.2) (layer "F.Cu") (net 11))
 (segment (start 186 91.67) (end 191.552081 91.67) (width 0.3) (layer "F.Cu") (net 1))
 (segment (start 190.665 69.435) (end 190.665 71.19261) (width 0.3) (layer "F.Cu") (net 1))
 (segment (start 195.77 95.887919) (end 195.77 97.09) (width 0.3) (layer "F.Cu") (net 1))
 (segment (start 187.870327 73.987283) (end 187.870327 74.26) (width 0.3) (layer "F.Cu") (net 1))
 (segment (start 189.179239 67.940761) (end 189.179239 67.949239) (width 0.3) (layer "F.Cu") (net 1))
 (segment (start 191.552081 91.67) (end 195.77 95.887919) (width 0.3) (layer "F.Cu") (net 1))
 (segment (start 189.179239 67.949239) (end 190.665 69.435) (width 0.3) (layer "F.Cu") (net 1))
 (segment (start 184.64 93.03) (end 186 91.67) (width 0.3) (layer "F.Cu") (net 1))
 (segment (start 187.870327 73.987283) (end 187.870327 89.799673) (width 0.3) (layer "F.Cu") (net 1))
 (segment (start 190.665 71.19261) (end 187.870327 73.987283) (width 0.3) (layer "F.Cu") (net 1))
 (segment (start 185.501522 71.618478) (end 187.870327 73.987283) (width 0.3) (layer "F.Cu") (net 1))
 (segment (start 187.870327 89.799673) (end 186 91.67) (width 0.3) (layer "F.Cu") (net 1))
 (segment (start 184.64 94.375) (end 184.64 93.03) (width 0.3) (layer "F.Cu") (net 1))
 (segment (start 195.68 97.09) (end 195.77 97.09) (width 0.2) (layer "B.Cu") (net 1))
 (segment (start 209.4 94.325) (end 209.4 91.6) (width 0.2) (layer "F.Cu") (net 8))
 (segment (start 208.160212 90.360212) (end 208.160212 66.470412) (width 0.2) (layer "F.Cu") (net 8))
 (segment (start 208.1449 66.4551) (end 208.1602 66.4551) (width 0.2) (layer "F.Cu") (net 8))
 (segment (start 209.45 94.375) (end 209.4 94.325) (width 0.2) (layer "F.Cu") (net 8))
 (segment (start 208.160212 66.470412) (end 208.1449 66.4551) (width 0.2) (layer "F.Cu") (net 8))
 (segment (start 209.4 91.6) (end 208.160212 90.360212) (width 0.2) (layer "F.Cu") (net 8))
 (segment (start 187.94 98.6019) (end 187.588 98.9539) (width 0.2) (layer "F.Cu") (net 13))
 (segment (start 209.95255 68.24745) (end 209.03 69.17) (width 0.2) (layer "F.Cu") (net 9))
 (segment (start 209.9602 68.2551) (end 209.95255 68.24745) (width 0.2) (layer "F.Cu") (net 9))
 (segment (start 209.03 90.03) (end 210.45 91.45) (width 0.2) (layer "F.Cu") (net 9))
 (segment (start 210.45 91.45) (end 210.45 94.375) (width 0.2) (layer "F.Cu") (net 9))
 (segment (start 209.03 69.17) (end 209.03 90.03) (width 0.2) (layer "F.Cu") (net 9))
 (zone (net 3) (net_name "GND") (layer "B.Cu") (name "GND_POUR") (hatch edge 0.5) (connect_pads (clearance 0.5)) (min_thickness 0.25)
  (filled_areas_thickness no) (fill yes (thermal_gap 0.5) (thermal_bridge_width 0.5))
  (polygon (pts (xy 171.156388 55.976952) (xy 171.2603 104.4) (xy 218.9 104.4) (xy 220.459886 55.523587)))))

